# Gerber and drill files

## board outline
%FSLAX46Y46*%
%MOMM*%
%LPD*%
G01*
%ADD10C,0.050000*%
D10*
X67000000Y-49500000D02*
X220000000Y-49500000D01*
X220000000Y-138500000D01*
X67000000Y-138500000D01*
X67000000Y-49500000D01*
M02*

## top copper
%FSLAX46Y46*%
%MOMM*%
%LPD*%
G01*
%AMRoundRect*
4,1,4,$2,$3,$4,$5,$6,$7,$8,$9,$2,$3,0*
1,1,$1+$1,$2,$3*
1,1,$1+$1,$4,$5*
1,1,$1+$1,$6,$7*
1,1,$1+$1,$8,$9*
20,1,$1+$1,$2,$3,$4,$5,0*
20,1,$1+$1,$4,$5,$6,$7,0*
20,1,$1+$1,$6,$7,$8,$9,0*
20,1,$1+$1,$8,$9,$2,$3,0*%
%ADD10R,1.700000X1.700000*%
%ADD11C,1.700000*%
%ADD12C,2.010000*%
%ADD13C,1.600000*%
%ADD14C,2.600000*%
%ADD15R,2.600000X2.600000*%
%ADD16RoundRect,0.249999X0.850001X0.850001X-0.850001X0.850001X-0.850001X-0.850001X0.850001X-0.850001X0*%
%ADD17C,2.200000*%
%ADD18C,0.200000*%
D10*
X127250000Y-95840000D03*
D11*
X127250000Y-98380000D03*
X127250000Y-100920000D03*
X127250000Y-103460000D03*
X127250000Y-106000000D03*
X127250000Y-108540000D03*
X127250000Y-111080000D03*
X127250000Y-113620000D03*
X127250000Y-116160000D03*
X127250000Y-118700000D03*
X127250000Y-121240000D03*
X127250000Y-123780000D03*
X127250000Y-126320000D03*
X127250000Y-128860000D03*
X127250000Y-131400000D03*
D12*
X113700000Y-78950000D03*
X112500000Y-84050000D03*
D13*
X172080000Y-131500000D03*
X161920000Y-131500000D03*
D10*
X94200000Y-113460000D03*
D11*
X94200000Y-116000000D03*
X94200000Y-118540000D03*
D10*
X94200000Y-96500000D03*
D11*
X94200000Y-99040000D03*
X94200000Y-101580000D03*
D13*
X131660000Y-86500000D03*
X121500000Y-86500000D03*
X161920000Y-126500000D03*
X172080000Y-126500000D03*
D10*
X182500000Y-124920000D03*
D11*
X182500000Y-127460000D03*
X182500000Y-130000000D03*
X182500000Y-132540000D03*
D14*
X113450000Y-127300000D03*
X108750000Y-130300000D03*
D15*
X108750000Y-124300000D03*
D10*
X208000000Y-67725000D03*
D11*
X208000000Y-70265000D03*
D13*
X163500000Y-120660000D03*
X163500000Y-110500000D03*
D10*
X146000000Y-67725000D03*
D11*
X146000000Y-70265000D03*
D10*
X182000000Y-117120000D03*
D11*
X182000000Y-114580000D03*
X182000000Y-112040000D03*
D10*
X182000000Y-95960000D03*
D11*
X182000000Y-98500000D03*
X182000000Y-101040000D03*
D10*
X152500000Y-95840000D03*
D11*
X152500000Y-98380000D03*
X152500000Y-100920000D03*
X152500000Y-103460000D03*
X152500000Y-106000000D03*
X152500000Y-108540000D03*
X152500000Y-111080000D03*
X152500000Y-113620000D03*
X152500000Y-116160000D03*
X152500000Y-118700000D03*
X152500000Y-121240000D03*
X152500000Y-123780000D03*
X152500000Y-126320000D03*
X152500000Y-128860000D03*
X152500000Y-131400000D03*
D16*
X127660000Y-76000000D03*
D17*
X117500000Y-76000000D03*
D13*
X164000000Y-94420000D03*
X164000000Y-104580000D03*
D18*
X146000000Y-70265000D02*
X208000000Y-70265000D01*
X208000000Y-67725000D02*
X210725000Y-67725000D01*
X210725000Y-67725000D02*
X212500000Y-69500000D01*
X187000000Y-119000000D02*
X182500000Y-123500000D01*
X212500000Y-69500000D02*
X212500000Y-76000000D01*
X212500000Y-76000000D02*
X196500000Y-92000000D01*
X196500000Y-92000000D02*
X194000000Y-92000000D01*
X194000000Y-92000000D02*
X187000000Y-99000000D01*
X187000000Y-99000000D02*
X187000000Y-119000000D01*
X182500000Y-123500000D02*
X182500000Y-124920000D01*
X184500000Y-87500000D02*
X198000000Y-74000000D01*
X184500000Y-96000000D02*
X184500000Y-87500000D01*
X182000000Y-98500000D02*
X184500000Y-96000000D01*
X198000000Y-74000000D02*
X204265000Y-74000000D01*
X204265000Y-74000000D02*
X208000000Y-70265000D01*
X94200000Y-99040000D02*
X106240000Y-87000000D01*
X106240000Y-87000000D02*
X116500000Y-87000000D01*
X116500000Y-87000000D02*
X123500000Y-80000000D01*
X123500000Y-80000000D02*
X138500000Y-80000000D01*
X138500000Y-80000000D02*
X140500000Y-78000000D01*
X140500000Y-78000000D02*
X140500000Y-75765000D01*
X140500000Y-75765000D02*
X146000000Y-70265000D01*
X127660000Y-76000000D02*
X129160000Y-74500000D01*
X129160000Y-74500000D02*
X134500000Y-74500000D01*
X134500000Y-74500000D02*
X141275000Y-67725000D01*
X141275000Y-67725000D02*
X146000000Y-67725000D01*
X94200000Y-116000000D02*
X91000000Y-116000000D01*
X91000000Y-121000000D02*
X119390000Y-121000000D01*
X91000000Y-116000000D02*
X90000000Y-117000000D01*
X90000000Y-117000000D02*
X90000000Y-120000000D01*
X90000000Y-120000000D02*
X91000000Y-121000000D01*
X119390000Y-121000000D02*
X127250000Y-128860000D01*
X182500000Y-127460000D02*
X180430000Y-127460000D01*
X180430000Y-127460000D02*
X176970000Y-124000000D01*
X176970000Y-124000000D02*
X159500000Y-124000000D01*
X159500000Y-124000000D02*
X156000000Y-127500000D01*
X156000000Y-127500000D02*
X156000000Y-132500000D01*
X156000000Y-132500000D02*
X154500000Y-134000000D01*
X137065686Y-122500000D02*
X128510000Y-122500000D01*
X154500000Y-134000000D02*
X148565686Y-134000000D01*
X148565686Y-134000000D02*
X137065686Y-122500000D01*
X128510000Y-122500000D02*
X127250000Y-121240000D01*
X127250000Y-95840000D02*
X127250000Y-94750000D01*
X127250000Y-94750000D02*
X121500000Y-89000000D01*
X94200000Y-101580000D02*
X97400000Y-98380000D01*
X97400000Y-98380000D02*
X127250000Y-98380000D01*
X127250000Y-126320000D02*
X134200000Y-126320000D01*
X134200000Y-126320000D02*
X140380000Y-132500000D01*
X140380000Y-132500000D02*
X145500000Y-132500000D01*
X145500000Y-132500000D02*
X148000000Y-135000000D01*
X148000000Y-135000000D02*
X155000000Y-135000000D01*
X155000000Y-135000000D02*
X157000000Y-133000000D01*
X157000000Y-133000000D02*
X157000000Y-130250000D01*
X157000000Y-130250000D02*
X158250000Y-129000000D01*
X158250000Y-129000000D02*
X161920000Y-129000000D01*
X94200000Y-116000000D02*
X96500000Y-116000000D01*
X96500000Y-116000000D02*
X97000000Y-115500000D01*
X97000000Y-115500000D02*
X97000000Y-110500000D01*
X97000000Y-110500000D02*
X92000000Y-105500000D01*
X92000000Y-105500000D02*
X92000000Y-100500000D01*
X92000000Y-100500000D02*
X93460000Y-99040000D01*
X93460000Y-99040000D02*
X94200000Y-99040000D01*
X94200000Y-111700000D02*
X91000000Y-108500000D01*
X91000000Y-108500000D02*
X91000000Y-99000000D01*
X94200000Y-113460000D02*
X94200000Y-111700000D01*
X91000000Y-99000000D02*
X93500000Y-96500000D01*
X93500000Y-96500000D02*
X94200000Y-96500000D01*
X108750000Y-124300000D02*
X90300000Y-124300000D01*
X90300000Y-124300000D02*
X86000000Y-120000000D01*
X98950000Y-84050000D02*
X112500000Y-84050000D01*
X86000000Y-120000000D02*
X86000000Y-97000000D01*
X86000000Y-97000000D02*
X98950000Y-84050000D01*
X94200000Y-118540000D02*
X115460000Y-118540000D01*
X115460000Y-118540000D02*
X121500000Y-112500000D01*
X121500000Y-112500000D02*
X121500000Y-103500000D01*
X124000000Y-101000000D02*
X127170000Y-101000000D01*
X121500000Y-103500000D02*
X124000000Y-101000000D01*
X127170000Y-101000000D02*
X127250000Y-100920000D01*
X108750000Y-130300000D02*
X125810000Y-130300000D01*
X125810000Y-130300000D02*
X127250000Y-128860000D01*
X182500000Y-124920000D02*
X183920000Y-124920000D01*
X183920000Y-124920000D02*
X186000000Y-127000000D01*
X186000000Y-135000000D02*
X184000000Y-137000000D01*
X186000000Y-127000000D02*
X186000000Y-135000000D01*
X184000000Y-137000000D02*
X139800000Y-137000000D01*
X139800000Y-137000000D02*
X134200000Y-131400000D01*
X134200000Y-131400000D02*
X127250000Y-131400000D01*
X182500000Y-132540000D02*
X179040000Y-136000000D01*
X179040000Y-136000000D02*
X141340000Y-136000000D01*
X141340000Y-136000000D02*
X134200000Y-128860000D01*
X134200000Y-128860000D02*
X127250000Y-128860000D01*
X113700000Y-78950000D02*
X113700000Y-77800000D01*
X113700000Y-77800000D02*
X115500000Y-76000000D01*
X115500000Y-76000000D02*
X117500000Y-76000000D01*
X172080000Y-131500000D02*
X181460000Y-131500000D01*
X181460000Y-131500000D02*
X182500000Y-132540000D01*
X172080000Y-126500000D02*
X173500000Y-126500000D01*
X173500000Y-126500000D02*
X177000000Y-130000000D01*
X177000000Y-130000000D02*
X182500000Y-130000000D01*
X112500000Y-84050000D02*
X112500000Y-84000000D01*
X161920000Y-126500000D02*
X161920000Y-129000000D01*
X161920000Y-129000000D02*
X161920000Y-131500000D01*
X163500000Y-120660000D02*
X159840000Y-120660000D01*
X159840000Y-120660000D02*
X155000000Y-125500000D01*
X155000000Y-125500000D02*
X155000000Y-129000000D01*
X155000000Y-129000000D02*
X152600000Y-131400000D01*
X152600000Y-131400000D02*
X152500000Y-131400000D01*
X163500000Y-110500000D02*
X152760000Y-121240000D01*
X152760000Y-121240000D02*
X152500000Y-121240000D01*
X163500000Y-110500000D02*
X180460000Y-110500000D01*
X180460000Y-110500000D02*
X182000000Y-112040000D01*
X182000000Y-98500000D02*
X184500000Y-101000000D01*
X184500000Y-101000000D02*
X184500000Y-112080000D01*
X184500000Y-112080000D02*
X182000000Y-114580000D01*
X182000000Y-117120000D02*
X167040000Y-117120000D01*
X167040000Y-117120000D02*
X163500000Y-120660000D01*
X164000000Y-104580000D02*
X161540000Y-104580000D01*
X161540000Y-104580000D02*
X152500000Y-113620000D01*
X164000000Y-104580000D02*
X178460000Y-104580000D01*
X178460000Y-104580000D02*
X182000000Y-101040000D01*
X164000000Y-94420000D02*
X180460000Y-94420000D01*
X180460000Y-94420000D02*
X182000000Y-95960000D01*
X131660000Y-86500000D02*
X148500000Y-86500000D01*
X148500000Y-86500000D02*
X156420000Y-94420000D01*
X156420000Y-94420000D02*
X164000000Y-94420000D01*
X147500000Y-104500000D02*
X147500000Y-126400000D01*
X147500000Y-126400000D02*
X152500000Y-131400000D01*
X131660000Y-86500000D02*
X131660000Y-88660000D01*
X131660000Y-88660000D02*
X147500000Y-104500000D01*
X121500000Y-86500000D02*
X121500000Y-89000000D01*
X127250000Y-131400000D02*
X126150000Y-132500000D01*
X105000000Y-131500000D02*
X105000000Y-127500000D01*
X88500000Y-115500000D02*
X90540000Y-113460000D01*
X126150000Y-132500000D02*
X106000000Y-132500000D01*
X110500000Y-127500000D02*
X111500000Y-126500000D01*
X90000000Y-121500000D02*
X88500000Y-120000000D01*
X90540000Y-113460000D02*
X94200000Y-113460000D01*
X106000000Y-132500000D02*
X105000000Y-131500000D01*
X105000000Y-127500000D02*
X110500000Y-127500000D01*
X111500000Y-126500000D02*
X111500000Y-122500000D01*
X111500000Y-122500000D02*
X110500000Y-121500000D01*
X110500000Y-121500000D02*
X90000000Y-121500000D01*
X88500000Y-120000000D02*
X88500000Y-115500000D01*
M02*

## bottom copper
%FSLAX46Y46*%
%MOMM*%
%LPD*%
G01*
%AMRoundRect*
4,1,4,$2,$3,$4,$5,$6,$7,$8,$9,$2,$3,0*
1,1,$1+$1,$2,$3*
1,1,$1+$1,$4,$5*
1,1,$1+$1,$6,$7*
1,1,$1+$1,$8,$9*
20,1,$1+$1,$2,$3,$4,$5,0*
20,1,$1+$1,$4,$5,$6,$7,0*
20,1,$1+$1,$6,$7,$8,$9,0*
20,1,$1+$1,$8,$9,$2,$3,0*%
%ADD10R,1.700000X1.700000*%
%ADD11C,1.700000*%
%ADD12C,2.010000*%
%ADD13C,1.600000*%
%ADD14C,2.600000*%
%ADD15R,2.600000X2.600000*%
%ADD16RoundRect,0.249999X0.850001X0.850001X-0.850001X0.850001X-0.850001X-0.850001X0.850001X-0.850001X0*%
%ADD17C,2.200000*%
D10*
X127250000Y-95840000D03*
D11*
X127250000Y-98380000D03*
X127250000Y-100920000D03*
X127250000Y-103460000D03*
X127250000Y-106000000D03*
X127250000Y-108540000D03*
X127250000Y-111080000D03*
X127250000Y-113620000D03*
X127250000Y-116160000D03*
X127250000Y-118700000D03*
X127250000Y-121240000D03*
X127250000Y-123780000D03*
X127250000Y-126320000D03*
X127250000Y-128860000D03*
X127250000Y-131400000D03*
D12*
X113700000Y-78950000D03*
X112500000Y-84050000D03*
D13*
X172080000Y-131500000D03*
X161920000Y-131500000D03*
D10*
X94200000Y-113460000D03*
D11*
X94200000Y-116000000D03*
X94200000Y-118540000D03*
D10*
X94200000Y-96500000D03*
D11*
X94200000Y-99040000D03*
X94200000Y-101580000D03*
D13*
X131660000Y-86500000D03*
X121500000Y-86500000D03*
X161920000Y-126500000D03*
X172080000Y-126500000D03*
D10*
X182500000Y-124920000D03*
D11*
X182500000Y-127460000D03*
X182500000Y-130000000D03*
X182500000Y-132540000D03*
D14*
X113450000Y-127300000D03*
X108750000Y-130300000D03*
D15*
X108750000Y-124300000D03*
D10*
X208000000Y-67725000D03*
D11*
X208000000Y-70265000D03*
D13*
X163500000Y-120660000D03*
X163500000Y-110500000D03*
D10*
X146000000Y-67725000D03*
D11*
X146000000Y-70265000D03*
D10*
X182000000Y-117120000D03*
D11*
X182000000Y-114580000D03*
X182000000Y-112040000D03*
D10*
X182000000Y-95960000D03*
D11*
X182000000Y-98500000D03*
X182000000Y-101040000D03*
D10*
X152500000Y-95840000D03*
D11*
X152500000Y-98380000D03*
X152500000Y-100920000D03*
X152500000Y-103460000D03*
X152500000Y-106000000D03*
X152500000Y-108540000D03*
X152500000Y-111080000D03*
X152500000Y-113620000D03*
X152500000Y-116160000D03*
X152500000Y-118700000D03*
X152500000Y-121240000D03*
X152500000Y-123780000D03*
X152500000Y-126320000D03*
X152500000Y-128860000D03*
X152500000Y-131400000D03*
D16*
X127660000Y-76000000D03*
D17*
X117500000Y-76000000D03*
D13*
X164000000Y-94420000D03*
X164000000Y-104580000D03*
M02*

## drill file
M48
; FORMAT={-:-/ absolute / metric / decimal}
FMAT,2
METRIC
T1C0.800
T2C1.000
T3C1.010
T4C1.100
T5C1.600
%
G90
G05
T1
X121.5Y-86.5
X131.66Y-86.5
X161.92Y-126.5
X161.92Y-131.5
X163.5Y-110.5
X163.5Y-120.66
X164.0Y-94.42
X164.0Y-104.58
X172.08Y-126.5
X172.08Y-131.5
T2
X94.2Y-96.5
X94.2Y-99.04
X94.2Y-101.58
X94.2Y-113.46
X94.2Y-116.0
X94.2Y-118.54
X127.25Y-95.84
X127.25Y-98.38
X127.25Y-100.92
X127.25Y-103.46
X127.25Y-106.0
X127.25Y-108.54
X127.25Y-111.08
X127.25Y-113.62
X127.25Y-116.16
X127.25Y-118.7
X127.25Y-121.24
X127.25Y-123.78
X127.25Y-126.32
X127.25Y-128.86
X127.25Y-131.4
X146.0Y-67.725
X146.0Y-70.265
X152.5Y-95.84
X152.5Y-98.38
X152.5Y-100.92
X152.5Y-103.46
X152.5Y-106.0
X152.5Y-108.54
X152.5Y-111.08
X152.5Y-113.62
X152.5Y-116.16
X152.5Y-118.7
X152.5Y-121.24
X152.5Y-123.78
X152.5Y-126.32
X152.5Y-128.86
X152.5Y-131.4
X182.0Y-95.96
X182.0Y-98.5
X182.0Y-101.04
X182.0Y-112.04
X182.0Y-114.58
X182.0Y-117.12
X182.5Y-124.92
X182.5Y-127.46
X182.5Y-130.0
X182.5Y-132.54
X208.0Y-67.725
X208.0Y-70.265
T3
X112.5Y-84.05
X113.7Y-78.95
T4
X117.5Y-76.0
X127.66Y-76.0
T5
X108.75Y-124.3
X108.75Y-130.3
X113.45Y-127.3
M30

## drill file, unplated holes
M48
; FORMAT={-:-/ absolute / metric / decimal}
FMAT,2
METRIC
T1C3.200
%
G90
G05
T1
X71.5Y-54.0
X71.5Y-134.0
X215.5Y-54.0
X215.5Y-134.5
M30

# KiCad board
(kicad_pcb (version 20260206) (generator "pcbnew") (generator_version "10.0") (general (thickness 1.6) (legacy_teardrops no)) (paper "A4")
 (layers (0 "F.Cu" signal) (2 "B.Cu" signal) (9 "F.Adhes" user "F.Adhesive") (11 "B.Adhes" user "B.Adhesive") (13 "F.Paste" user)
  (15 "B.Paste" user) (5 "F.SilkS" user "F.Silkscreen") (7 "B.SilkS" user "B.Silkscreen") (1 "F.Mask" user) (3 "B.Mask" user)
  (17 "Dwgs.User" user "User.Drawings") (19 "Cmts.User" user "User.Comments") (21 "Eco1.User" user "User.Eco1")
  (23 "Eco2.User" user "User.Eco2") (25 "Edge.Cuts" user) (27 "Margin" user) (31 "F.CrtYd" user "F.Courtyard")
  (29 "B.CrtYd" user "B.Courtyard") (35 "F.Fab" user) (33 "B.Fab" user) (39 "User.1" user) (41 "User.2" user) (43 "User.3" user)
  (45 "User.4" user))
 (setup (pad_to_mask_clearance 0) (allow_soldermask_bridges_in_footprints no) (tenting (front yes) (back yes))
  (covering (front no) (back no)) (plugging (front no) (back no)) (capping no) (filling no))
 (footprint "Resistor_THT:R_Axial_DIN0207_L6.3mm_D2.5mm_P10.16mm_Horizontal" (layer "F.Cu") (at 161.92 126.5)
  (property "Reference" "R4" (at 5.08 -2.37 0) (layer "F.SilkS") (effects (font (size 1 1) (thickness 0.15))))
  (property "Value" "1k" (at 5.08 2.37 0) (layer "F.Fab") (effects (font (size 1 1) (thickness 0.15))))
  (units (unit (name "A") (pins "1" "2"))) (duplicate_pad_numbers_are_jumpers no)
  (pad "1" thru_hole circle (at 0 0) (size 1.6 1.6) (drill 0.8) (layers "*.Cu" "*.Mask") (remove_unused_layers no) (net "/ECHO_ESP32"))
  (pad "2" thru_hole circle (at 10.16 0) (size 1.6 1.6) (drill 0.8) (layers "*.Cu" "*.Mask") (remove_unused_layers no) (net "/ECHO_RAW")))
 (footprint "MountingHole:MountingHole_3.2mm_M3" (layer "F.Cu") (at 215.5 134.5)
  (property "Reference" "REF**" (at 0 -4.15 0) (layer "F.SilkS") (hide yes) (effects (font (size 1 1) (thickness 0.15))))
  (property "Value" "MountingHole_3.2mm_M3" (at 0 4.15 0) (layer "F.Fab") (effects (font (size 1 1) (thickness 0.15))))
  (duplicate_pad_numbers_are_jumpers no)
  (pad "" np_thru_hole circle (at 0 0) (size 3.2 3.2) (drill 3.2) (layers "*.Cu" "*.Mask")))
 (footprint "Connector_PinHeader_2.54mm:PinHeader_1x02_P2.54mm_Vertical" (layer "F.Cu") (at 208 67.725)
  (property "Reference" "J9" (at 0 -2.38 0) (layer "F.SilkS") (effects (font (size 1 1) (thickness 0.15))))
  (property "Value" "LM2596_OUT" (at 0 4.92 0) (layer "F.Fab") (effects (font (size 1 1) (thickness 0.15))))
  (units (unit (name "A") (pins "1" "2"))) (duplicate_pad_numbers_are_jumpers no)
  (pad "1" thru_hole rect (at 0 0) (size 1.7 1.7) (drill 1) (layers "*.Cu" "*.Mask") (remove_unused_layers no) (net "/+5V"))
  (pad "2" thru_hole circle (at 0 2.54) (size 1.7 1.7) (drill 1) (layers "*.Cu" "*.Mask") (remove_unused_layers no) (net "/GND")))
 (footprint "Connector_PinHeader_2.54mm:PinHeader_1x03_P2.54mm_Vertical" (layer "F.Cu") (at 94.2 113.46)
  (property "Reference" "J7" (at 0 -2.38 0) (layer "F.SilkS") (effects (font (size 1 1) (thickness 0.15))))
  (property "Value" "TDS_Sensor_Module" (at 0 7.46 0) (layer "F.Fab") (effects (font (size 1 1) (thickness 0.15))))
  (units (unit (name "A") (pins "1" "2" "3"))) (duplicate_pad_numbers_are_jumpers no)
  (pad "1" thru_hole rect (at 0 0) (size 1.7 1.7) (drill 1) (layers "*.Cu" "*.Mask") (remove_unused_layers no) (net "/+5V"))
  (pad "2" thru_hole circle (at 0 2.54) (size 1.7 1.7) (drill 1) (layers "*.Cu" "*.Mask") (remove_unused_layers no) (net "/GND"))
  (pad "3" thru_hole circle (at 0 5.08) (size 1.7 1.7) (drill 1) (layers "*.Cu" "*.Mask") (remove_unused_layers no) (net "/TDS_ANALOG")))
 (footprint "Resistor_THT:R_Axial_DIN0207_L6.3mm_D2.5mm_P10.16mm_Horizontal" (layer "F.Cu") (at 131.66 86.5 180)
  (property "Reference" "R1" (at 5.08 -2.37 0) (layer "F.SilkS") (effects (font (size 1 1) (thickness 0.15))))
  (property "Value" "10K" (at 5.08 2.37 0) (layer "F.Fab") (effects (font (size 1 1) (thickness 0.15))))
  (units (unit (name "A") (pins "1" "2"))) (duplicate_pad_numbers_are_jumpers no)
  (pad "1" thru_hole circle (at 0 0 180) (size 1.6 1.6) (drill 0.8) (layers "*.Cu" "*.Mask") (remove_unused_layers no) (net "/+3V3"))
  (pad "2" thru_hole circle (at 10.16 0 180) (size 1.6 1.6) (drill 0.8) (layers "*.Cu" "*.Mask") (remove_unused_layers no) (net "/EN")))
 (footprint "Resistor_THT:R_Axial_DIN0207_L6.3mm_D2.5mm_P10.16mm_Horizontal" (layer "F.Cu") (at 163.5 120.66 90)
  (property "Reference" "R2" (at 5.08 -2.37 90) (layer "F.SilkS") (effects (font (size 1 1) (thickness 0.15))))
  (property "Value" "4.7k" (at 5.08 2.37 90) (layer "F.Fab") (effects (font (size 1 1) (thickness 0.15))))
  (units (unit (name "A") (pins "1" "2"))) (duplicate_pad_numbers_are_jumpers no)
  (pad "1" thru_hole circle (at 0 0 90) (size 1.6 1.6) (drill 0.8) (layers "*.Cu" "*.Mask") (remove_unused_layers no) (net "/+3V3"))
  (pad "2" thru_hole circle (at 10.16 0 90) (size 1.6 1.6) (drill 0.8) (layers "*.Cu" "*.Mask") (remove_unused_layers no)
   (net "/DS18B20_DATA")))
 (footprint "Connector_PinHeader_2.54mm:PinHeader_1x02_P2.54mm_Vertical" (layer "F.Cu") (at 146 67.725)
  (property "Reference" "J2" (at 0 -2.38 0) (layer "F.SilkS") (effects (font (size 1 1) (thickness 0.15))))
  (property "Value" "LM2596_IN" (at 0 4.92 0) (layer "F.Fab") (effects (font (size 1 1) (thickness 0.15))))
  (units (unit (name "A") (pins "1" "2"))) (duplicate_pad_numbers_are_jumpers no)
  (pad "1" thru_hole rect (at 0 0) (size 1.7 1.7) (drill 1) (layers "*.Cu" "*.Mask") (remove_unused_layers no) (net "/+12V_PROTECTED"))
  (pad "2" thru_hole circle (at 0 2.54) (size 1.7 1.7) (drill 1) (layers "*.Cu" "*.Mask") (remove_unused_layers no) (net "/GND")))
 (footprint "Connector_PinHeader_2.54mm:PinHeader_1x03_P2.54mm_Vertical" (layer "F.Cu") (at 182 117.12 180)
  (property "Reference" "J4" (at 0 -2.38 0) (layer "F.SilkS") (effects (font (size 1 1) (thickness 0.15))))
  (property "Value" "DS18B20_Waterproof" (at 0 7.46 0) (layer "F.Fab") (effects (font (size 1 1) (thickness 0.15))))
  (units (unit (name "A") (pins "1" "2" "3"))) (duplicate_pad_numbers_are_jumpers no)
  (pad "1" thru_hole rect (at 0 0 180) (size 1.7 1.7) (drill 1) (layers "*.Cu" "*.Mask") (remove_unused_layers no) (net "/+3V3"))
  (pad "2" thru_hole circle (at 0 2.54 180) (size 1.7 1.7) (drill 1) (layers "*.Cu" "*.Mask") (remove_unused_layers no) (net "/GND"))
  (pad "3" thru_hole circle (at 0 5.08 180) (size 1.7 1.7) (drill 1) (layers "*.Cu" "*.Mask") (remove_unused_layers no)
   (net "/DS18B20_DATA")))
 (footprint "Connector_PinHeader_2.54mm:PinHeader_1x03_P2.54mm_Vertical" (layer "F.Cu") (at 94.2 96.5)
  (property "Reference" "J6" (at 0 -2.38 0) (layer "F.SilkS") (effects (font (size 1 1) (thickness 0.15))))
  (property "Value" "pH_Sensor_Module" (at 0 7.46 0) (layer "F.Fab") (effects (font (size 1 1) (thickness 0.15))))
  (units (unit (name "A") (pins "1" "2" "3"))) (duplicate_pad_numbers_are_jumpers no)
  (pad "1" thru_hole rect (at 0 0) (size 1.7 1.7) (drill 1) (layers "*.Cu" "*.Mask") (remove_unused_layers no) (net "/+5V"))
  (pad "2" thru_hole circle (at 0 2.54) (size 1.7 1.7) (drill 1) (layers "*.Cu" "*.Mask") (remove_unused_layers no) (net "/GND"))
  (pad "3" thru_hole circle (at 0 5.08) (size 1.7 1.7) (drill 1) (layers "*.Cu" "*.Mask") (remove_unused_layers no) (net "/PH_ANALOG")))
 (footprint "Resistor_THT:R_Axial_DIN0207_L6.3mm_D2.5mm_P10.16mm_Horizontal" (layer "F.Cu") (at 161.92 131.5)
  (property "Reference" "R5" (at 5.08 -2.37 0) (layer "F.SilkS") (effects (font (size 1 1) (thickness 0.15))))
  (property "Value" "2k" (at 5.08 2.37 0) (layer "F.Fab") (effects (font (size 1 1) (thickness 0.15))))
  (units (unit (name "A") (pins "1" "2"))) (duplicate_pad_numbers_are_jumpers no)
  (pad "1" thru_hole circle (at 0 0) (size 1.6 1.6) (drill 0.8) (layers "*.Cu" "*.Mask") (remove_unused_layers no) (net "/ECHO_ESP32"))
  (pad "2" thru_hole circle (at 10.16 0) (size 1.6 1.6) (drill 0.8) (layers "*.Cu" "*.Mask") (remove_unused_layers no) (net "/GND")))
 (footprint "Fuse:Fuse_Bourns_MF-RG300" (layer "F.Cu") (at 113.7 78.95 -90)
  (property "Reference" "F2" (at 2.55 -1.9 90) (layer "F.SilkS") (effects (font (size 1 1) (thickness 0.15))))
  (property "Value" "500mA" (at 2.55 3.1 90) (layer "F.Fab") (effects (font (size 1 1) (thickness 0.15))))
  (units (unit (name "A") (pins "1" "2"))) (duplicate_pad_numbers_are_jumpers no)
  (pad "1" thru_hole circle (at 0 0 270) (size 2.01 2.01) (drill 1.01) (layers "*.Cu" "*.Mask") (remove_unused_layers no)
   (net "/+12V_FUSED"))
  (pad "2" thru_hole circle (at 5.1 1.2 270) (size 2.01 2.01) (drill 1.01) (layers "*.Cu" "*.Mask") (remove_unused_layers no)
   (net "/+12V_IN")))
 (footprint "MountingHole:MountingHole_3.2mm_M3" (layer "F.Cu") (at 71.5 134)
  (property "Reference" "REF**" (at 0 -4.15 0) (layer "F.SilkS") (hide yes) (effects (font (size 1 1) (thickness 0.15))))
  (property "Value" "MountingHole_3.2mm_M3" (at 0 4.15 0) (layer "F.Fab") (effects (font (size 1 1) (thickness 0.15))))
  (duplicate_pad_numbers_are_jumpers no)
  (pad "" np_thru_hole circle (at 0 0) (size 3.2 3.2) (drill 3.2) (layers "*.Cu" "*.Mask")))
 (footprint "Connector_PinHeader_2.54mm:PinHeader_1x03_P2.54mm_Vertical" (layer "F.Cu") (at 182 95.96)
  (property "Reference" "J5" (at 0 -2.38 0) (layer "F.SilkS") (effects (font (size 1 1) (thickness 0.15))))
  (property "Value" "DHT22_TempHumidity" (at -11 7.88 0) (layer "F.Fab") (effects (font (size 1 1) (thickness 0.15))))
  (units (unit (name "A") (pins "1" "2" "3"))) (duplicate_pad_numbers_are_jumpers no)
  (pad "1" thru_hole rect (at 0 0) (size 1.7 1.7) (drill 1) (layers "*.Cu" "*.Mask") (remove_unused_layers no) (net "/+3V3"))
  (pad "2" thru_hole circle (at 0 2.54) (size 1.7 1.7) (drill 1) (layers "*.Cu" "*.Mask") (remove_unused_layers no) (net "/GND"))
  (pad "3" thru_hole circle (at 0 5.08) (size 1.7 1.7) (drill 1) (layers "*.Cu" "*.Mask") (remove_unused_layers no) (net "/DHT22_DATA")))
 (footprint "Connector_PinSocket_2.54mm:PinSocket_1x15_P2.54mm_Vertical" (layer "F.Cu") (at 127.25 95.84)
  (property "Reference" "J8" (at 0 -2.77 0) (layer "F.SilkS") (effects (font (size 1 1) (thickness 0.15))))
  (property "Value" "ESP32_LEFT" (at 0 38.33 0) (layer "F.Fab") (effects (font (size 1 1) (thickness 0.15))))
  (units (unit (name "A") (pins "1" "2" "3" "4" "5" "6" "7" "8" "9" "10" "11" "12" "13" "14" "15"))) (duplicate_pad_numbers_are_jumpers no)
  (pad "1" thru_hole rect (at 0 0) (size 1.7 1.7) (drill 1) (layers "*.Cu" "*.Mask") (remove_unused_layers no) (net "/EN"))
  (pad "2" thru_hole circle (at 0 2.54) (size 1.7 1.7) (drill 1) (layers "*.Cu" "*.Mask") (remove_unused_layers no) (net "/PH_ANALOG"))
  (pad "3" thru_hole circle (at 0 5.08) (size 1.7 1.7) (drill 1) (layers "*.Cu" "*.Mask") (remove_unused_layers no) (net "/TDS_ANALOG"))
  (pad "4" thru_hole circle (at 0 7.62) (size 1.7 1.7) (drill 1) (layers "*.Cu" "*.Mask") (remove_unused_layers no)
   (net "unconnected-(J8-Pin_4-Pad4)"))
  (pad "5" thru_hole circle (at 0 10.16) (size 1.7 1.7) (drill 1) (layers "*.Cu" "*.Mask") (remove_unused_layers no)
   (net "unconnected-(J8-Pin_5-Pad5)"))
  (pad "6" thru_hole circle (at 0 12.7) (size 1.7 1.7) (drill 1) (layers "*.Cu" "*.Mask") (remove_unused_layers no)
   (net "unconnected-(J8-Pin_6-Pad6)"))
  (pad "7" thru_hole circle (at 0 15.24) (size 1.7 1.7) (drill 1) (layers "*.Cu" "*.Mask") (remove_unused_layers no)
   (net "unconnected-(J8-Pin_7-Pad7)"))
  (pad "8" thru_hole circle (at 0 17.78) (size 1.7 1.7) (drill 1) (layers "*.Cu" "*.Mask") (remove_unused_layers no)
   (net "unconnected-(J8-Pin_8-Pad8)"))
  (pad "9" thru_hole circle (at 0 20.32) (size 1.7 1.7) (drill 1) (layers "*.Cu" "*.Mask") (remove_unused_layers no)
   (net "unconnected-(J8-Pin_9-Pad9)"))
  (pad "10" thru_hole circle (at 0 22.86) (size 1.7 1.7) (drill 1) (layers "*.Cu" "*.Mask") (remove_unused_layers no)
   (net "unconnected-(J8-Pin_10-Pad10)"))
  (pad "11" thru_hole circle (at 0 25.4) (size 1.7 1.7) (drill 1) (layers "*.Cu" "*.Mask") (remove_unused_layers no) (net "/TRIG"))
  (pad "12" thru_hole circle (at 0 27.94) (size 1.7 1.7) (drill 1) (layers "*.Cu" "*.Mask") (remove_unused_layers no)
   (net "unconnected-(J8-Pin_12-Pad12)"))
  (pad "13" thru_hole circle (at 0 30.48) (size 1.7 1.7) (drill 1) (layers "*.Cu" "*.Mask") (remove_unused_layers no) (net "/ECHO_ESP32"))
  (pad "14" thru_hole circle (at 0 33.02) (size 1.7 1.7) (drill 1) (layers "*.Cu" "*.Mask") (remove_unused_layers no) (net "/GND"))
  (pad "15" thru_hole circle (at 0 35.56) (size 1.7 1.7) (drill 1) (layers "*.Cu" "*.Mask") (remove_unused_layers no) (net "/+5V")))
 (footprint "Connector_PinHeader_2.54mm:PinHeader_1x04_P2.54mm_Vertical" (layer "F.Cu") (at 182.5 124.92)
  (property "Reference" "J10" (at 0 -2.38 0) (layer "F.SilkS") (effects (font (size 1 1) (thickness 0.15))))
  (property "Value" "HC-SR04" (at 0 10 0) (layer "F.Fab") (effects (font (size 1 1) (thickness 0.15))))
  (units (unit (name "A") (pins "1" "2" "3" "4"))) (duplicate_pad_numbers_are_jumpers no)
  (pad "1" thru_hole rect (at 0 0) (size 1.7 1.7) (drill 1) (layers "*.Cu" "*.Mask") (remove_unused_layers no) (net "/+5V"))
  (pad "2" thru_hole circle (at 0 2.54) (size 1.7 1.7) (drill 1) (layers "*.Cu" "*.Mask") (remove_unused_layers no) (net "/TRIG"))
  (pad "3" thru_hole circle (at 0 5.08) (size 1.7 1.7) (drill 1) (layers "*.Cu" "*.Mask") (remove_unused_layers no) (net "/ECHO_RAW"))
  (pad "4" thru_hole circle (at 0 7.62) (size 1.7 1.7) (drill 1) (layers "*.Cu" "*.Mask") (remove_unused_layers no) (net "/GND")))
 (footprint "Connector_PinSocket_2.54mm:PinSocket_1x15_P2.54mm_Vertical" (layer "F.Cu") (at 152.5 95.84)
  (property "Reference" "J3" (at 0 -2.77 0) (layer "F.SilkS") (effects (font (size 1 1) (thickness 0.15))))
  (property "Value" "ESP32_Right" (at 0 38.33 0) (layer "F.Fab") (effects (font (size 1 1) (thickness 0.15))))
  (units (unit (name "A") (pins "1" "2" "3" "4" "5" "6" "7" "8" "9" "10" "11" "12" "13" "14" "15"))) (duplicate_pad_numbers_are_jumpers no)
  (pad "1" thru_hole rect (at 0 0) (size 1.7 1.7) (drill 1) (layers "*.Cu" "*.Mask") (remove_unused_layers no)
   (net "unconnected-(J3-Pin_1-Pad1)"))
  (pad "2" thru_hole circle (at 0 2.54) (size 1.7 1.7) (drill 1) (layers "*.Cu" "*.Mask") (remove_unused_layers no)
   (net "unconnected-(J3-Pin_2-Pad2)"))
  (pad "3" thru_hole circle (at 0 5.08) (size 1.7 1.7) (drill 1) (layers "*.Cu" "*.Mask") (remove_unused_layers no)
   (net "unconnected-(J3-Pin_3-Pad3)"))
  (pad "4" thru_hole circle (at 0 7.62) (size 1.7 1.7) (drill 1) (layers "*.Cu" "*.Mask") (remove_unused_layers no)
   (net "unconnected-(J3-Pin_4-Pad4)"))
  (pad "5" thru_hole circle (at 0 10.16) (size 1.7 1.7) (drill 1) (layers "*.Cu" "*.Mask") (remove_unused_layers no)
   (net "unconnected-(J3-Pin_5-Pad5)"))
  (pad "6" thru_hole circle (at 0 12.7) (size 1.7 1.7) (drill 1) (layers "*.Cu" "*.Mask") (remove_unused_layers no)
   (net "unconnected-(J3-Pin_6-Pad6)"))
  (pad "7" thru_hole circle (at 0 15.24) (size 1.7 1.7) (drill 1) (layers "*.Cu" "*.Mask") (remove_unused_layers no)
   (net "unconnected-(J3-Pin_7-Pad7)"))
  (pad "8" thru_hole circle (at 0 17.78) (size 1.7 1.7) (drill 1) (layers "*.Cu" "*.Mask") (remove_unused_layers no) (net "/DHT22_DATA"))
  (pad "9" thru_hole circle (at 0 20.32) (size 1.7 1.7) (drill 1) (layers "*.Cu" "*.Mask") (remove_unused_layers no)
   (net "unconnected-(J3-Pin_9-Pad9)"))
  (pad "10" thru_hole circle (at 0 22.86) (size 1.7 1.7) (drill 1) (layers "*.Cu" "*.Mask") (remove_unused_layers no)
   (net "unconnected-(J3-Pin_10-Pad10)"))
  (pad "11" thru_hole circle (at 0 25.4) (size 1.7 1.7) (drill 1) (layers "*.Cu" "*.Mask") (remove_unused_layers no) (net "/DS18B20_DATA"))
  (pad "12" thru_hole circle (at 0 27.94) (size 1.7 1.7) (drill 1) (layers "*.Cu" "*.Mask") (remove_unused_layers no)
   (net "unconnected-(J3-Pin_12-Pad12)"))
  (pad "13" thru_hole circle (at 0 30.48) (size 1.7 1.7) (drill 1) (layers "*.Cu" "*.Mask") (remove_unused_layers no)
   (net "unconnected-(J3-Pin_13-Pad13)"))
  (pad "14" thru_hole circle (at 0 33.02) (size 1.7 1.7) (drill 1) (layers "*.Cu" "*.Mask") (remove_unused_layers no)
   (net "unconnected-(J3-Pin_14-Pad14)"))
  (pad "15" thru_hole circle (at 0 35.56) (size 1.7 1.7) (drill 1) (layers "*.Cu" "*.Mask") (remove_unused_layers no) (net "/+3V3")))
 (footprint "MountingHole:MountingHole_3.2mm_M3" (layer "F.Cu") (at 215.5 54)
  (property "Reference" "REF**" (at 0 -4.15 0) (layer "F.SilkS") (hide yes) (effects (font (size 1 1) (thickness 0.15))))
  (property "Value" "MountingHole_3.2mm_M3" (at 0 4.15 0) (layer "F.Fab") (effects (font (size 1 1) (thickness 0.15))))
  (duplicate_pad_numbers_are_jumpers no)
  (pad "" np_thru_hole circle (at 0 0) (size 3.2 3.2) (drill 3.2) (layers "*.Cu" "*.Mask")))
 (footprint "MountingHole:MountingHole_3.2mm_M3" (layer "F.Cu") (at 71.5 54)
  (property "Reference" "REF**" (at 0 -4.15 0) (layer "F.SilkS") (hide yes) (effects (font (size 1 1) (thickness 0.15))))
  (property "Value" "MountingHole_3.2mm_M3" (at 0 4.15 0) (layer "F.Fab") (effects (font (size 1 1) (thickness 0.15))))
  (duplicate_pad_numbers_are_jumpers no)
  (pad "" np_thru_hole circle (at 0 0) (size 3.2 3.2) (drill 3.2) (layers "*.Cu" "*.Mask")))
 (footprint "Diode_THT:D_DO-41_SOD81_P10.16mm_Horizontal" (layer "F.Cu") (at 127.66 76 180)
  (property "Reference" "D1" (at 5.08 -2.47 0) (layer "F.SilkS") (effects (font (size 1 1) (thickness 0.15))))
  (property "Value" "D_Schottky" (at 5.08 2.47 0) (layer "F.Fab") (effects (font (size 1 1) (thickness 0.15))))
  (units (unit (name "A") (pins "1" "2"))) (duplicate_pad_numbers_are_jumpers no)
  (pad "1" thru_hole roundrect (at 0 0 180) (size 2.2 2.2) (drill 1.1) (layers "*.Cu" "*.Mask") (remove_unused_layers no)
   (roundrect_rratio 0.113636) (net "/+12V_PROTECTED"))
  (pad "2" thru_hole circle (at 10.16 0 180) (size 2.2 2.2) (drill 1.1) (layers "*.Cu" "*.Mask") (remove_unused_layers no)
   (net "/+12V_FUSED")))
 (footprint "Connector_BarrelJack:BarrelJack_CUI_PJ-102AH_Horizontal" (layer "F.Cu") (at 108.75 124.3)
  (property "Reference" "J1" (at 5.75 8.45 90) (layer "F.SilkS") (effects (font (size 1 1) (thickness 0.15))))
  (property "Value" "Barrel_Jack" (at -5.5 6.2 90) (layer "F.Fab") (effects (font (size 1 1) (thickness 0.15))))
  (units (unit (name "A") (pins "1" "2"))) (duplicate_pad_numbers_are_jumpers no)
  (pad "1" thru_hole rect (at 0 0) (size 2.6 2.6) (drill 1.6) (layers "*.Cu" "*.Mask") (remove_unused_layers no) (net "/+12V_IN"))
  (pad "2" thru_hole circle (at 0 6) (size 2.6 2.6) (drill 1.6) (layers "*.Cu" "*.Mask") (remove_unused_layers no) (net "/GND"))
  (pad "3" thru_hole circle (at 4.7 3) (size 2.6 2.6) (drill 1.6) (layers "*.Cu" "*.Mask") (remove_unused_layers no)))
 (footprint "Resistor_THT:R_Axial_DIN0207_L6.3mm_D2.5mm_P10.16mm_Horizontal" (layer "F.Cu") (at 164 94.42 -90)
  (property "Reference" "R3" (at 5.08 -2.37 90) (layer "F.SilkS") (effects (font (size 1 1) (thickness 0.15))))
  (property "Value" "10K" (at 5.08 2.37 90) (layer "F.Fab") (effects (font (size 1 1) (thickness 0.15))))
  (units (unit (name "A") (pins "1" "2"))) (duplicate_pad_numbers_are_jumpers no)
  (pad "1" thru_hole circle (at 0 0 270) (size 1.6 1.6) (drill 0.8) (layers "*.Cu" "*.Mask") (remove_unused_layers no) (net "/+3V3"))
  (pad "2" thru_hole circle (at 10.16 0 270) (size 1.6 1.6) (drill 0.8) (layers "*.Cu" "*.Mask") (remove_unused_layers no)
   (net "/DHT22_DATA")))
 (gr_rect (start 67 49.5) (end 220 138.5) (stroke (width 0.05) (type default)) (fill no) (layer "Edge.Cuts"))
 (segment (start 110.5 127.5) (end 111.5 126.5) (width 0.2) (layer "F.Cu") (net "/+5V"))
 (segment (start 212.5 69.5) (end 212.5 76) (width 0.2) (layer "F.Cu") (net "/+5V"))
 (segment (start 93.5 96.5) (end 94.2 96.5) (width 0.2) (layer "F.Cu") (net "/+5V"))
 (segment (start 111.5 122.5) (end 110.5 121.5) (width 0.2) (layer "F.Cu") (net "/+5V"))
 (segment (start 111.5 126.5) (end 111.5 122.5) (width 0.2) (layer "F.Cu") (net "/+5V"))
 (segment (start 186 135) (end 184 137) (width 0.2) (layer "F.Cu") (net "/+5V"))
 (segment (start 186 127) (end 186 135) (width 0.2) (layer "F.Cu") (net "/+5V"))
 (segment (start 139.8 137) (end 134.2 131.4) (width 0.2) (layer "F.Cu") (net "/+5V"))
 (segment (start 126.15 132.5) (end 106 132.5) (width 0.2) (layer "F.Cu") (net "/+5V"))
 (segment (start 212.5 76) (end 196.5 92) (width 0.2) (layer "F.Cu") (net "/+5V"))
 (segment (start 94.2 113.46) (end 94.2 111.7) (width 0.2) (layer "F.Cu") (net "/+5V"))
 (segment (start 105 131.5) (end 105 127.5) (width 0.2) (layer "F.Cu") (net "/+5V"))
 (segment (start 184 137) (end 139.8 137) (width 0.2) (layer "F.Cu") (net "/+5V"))
 (segment (start 88.5 115.5) (end 90.54 113.46) (width 0.2) (layer "F.Cu") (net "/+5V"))
 (segment (start 187 99) (end 187 119) (width 0.2) (layer "F.Cu") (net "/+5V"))
 (segment (start 90.54 113.46) (end 94.2 113.46) (width 0.2) (layer "F.Cu") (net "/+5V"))
 (segment (start 90 121.5) (end 88.5 120) (width 0.2) (layer "F.Cu") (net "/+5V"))
 (segment (start 94.2 111.7) (end 91 108.5) (width 0.2) (layer "F.Cu") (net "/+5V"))
 (segment (start 187 119) (end 182.5 123.5) (width 0.2) (layer "F.Cu") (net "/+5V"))
 (segment (start 91 99) (end 93.5 96.5) (width 0.2) (layer "F.Cu") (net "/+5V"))
 (segment (start 182.5 124.92) (end 183.92 124.92) (width 0.2) (layer "F.Cu") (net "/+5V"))
 (segment (start 91 108.5) (end 91 99) (width 0.2) (layer "F.Cu") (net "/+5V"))
 (segment (start 208 67.725) (end 210.725 67.725) (width 0.2) (layer "F.Cu") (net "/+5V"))
 (segment (start 110.5 121.5) (end 90 121.5) (width 0.2) (layer "F.Cu") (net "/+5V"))
 (segment (start 127.25 131.4) (end 126.15 132.5) (width 0.2) (layer "F.Cu") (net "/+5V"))
 (segment (start 105 127.5) (end 110.5 127.5) (width 0.2) (layer "F.Cu") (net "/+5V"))
 (segment (start 134.2 131.4) (end 127.25 131.4) (width 0.2) (layer "F.Cu") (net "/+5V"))
 (segment (start 196.5 92) (end 194 92) (width 0.2) (layer "F.Cu") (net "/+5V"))
 (segment (start 106 132.5) (end 105 131.5) (width 0.2) (layer "F.Cu") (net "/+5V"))
 (segment (start 194 92) (end 187 99) (width 0.2) (layer "F.Cu") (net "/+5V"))
 (segment (start 210.725 67.725) (end 212.5 69.5) (width 0.2) (layer "F.Cu") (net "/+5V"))
 (segment (start 88.5 120) (end 88.5 115.5) (width 0.2) (layer "F.Cu") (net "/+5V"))
 (segment (start 183.92 124.92) (end 186 127) (width 0.2) (layer "F.Cu") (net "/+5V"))
 (segment (start 182.5 123.5) (end 182.5 124.92) (width 0.2) (layer "F.Cu") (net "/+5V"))
 (segment (start 91 116) (end 90 117) (width 0.2) (layer "F.Cu") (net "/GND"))
 (segment (start 141.34 136) (end 134.2 128.86) (width 0.2) (layer "F.Cu") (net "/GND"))
 (segment (start 90 117) (end 90 120) (width 0.2) (layer "F.Cu") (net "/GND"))
 (segment (start 97 115.5) (end 97 110.5) (width 0.2) (layer "F.Cu") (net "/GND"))
 (segment (start 94.2 116) (end 91 116) (width 0.2) (layer "F.Cu") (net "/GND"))
 (segment (start 134.2 128.86) (end 127.25 128.86) (width 0.2) (layer "F.Cu") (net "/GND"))
 (segment (start 184.5 87.5) (end 198 74) (width 0.2) (layer "F.Cu") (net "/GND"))
 (segment (start 94.2 99.04) (end 106.24 87) (width 0.2) (layer "F.Cu") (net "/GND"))
 (segment (start 108.75 130.3) (end 125.81 130.3) (width 0.2) (layer "F.Cu") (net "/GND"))
 (segment (start 204.265 74) (end 208 70.265) (width 0.2) (layer "F.Cu") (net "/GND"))
 (segment (start 181.46 131.5) (end 182.5 132.54) (width 0.2) (layer "F.Cu") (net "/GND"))
 (segment (start 90 120) (end 91 121) (width 0.2) (layer "F.Cu") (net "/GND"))
 (segment (start 93.46 99.04) (end 94.2 99.04) (width 0.2) (layer "F.Cu") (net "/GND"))
 (segment (start 179.04 136) (end 141.34 136) (width 0.2) (layer "F.Cu") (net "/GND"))
 (segment (start 182.5 132.54) (end 179.04 136) (width 0.2) (layer "F.Cu") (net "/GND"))
 (segment (start 123.5 80) (end 138.5 80) (width 0.2) (layer "F.Cu") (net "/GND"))
 (segment (start 92 100.5) (end 93.46 99.04) (width 0.2) (layer "F.Cu") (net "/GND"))
 (segment (start 184.5 96) (end 184.5 87.5) (width 0.2) (layer "F.Cu") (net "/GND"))
 (segment (start 140.5 78) (end 140.5 75.765) (width 0.2) (layer "F.Cu") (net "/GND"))
 (segment (start 94.2 116) (end 96.5 116) (width 0.2) (layer "F.Cu") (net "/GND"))
 (segment (start 96.5 116) (end 97 115.5) (width 0.2) (layer "F.Cu") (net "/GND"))
 (segment (start 198 74) (end 204.265 74) (width 0.2) (layer "F.Cu") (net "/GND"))
 (segment (start 119.39 121) (end 127.25 128.86) (width 0.2) (layer "F.Cu") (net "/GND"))
 (segment (start 138.5 80) (end 140.5 78) (width 0.2) (layer "F.Cu") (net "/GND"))
 (segment (start 125.81 130.3) (end 127.25 128.86) (width 0.2) (layer "F.Cu") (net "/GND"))
 (segment (start 140.5 75.765) (end 146 70.265) (width 0.2) (layer "F.Cu") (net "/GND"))
 (segment (start 92 105.5) (end 92 100.5) (width 0.2) (layer "F.Cu") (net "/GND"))
 (segment (start 116.5 87) (end 123.5 80) (width 0.2) (layer "F.Cu") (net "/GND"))
 (segment (start 146 70.265) (end 208 70.265) (width 0.2) (layer "F.Cu") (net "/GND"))
 (segment (start 184.5 101) (end 184.5 112.08) (width 0.2) (layer "F.Cu") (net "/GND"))
 (segment (start 182 98.5) (end 184.5 101) (width 0.2) (layer "F.Cu") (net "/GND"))
 (segment (start 91 121) (end 119.39 121) (width 0.2) (layer "F.Cu") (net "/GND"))
 (segment (start 182 98.5) (end 184.5 96) (width 0.2) (layer "F.Cu") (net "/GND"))
 (segment (start 97 110.5) (end 92 105.5) (width 0.2) (layer "F.Cu") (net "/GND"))
 (segment (start 172.08 131.5) (end 181.46 131.5) (width 0.2) (layer "F.Cu") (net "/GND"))
 (segment (start 184.5 112.08) (end 182 114.58) (width 0.2) (layer "F.Cu") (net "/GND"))
 (segment (start 106.24 87) (end 116.5 87) (width 0.2) (layer "F.Cu") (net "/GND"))
 (segment (start 115.46 118.54) (end 121.5 112.5) (width 0.2) (layer "F.Cu") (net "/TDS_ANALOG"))
 (segment (start 94.2 118.54) (end 115.46 118.54) (width 0.2) (layer "F.Cu") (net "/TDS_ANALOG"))
 (segment (start 124 101) (end 127.17 101) (width 0.2) (layer "F.Cu") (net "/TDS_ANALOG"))
 (segment (start 127.17 101) (end 127.25 100.92) (width 0.2) (layer "F.Cu") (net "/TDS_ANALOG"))
 (segment (start 121.5 103.5) (end 124 101) (width 0.2) (layer "F.Cu") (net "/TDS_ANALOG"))
 (segment (start 121.5 112.5) (end 121.5 103.5) (width 0.2) (layer "F.Cu") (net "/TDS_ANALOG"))
 (segment (start 155 125.5) (end 155 129) (width 0.2) (layer "F.Cu") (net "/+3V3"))
 (segment (start 152.6 131.4) (end 152.5 131.4) (width 0.2) (layer "F.Cu") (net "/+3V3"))
 (segment (start 147.5 104.5) (end 147.5 126.4) (width 0.2) (layer "F.Cu") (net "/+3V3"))
 (segment (start 180.46 94.42) (end 182 95.96) (width 0.2) (layer "F.Cu") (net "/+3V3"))
 (segment (start 156.42 94.42) (end 164 94.42) (width 0.2) (layer "F.Cu") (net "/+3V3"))
 (segment (start 148.5 86.5) (end 156.42 94.42) (width 0.2) (layer "F.Cu") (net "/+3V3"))
 (segment (start 147.5 126.4) (end 152.5 131.4) (width 0.2) (layer "F.Cu") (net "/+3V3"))
 (segment (start 163.5 120.66) (end 159.84 120.66) (width 0.2) (layer "F.Cu") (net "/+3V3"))
 (segment (start 131.66 86.5) (end 148.5 86.5) (width 0.2) (layer "F.Cu") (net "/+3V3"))
 (segment (start 159.84 120.66) (end 155 125.5) (width 0.2) (layer "F.Cu") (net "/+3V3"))
 (segment (start 131.66 86.5) (end 131.66 88.66) (width 0.2) (layer "F.Cu") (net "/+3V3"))
 (segment (start 131.66 88.66) (end 147.5 104.5) (width 0.2) (layer "F.Cu") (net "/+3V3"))
 (segment (start 164 94.42) (end 180.46 94.42) (width 0.2) (layer "F.Cu") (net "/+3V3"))
 (segment (start 155 129) (end 152.6 131.4) (width 0.2) (layer "F.Cu") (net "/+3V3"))
 (segment (start 167.04 117.12) (end 163.5 120.66) (width 0.2) (layer "F.Cu") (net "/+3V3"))
 (segment (start 182 117.12) (end 167.04 117.12) (width 0.2) (layer "F.Cu") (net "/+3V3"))
 (segment (start 121.5 86.5) (end 121.5 89) (width 0.2) (layer "F.Cu") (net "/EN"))
 (segment (start 127.25 95.84) (end 127.25 94.75) (width 0.2) (layer "F.Cu") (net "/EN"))
 (segment (start 127.25 94.75) (end 121.5 89) (width 0.2) (layer "F.Cu") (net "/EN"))
 (segment (start 152.76 121.24) (end 152.5 121.24) (width 0.2) (layer "F.Cu") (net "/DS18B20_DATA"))
 (segment (start 180.46 110.5) (end 182 112.04) (width 0.2) (layer "F.Cu") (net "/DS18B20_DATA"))
 (segment (start 163.5 110.5) (end 180.46 110.5) (width 0.2) (layer "F.Cu") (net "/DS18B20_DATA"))
 (segment (start 163.5 110.5) (end 152.76 121.24) (width 0.2) (layer "F.Cu") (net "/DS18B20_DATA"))
 (segment (start 141.275 67.725) (end 146 67.725) (width 0.2) (layer "F.Cu") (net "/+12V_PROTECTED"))
 (segment (start 134.5 74.5) (end 141.275 67.725) (width 0.2) (layer "F.Cu") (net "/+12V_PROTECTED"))
 (segment (start 127.66 76) (end 129.16 74.5) (width 0.2) (layer "F.Cu") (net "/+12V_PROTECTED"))
 (segment (start 129.16 74.5) (end 134.5 74.5) (width 0.2) (layer "F.Cu") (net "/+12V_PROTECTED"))
 (segment (start 97.4 98.38) (end 127.25 98.38) (width 0.2) (layer "F.Cu") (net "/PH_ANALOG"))
 (segment (start 94.2 101.58) (end 97.4 98.38) (width 0.2) (layer "F.Cu") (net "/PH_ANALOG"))
 (segment (start 115.5 76) (end 117.5 76) (width 0.2) (layer "F.Cu") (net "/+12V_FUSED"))
 (segment (start 113.7 78.95) (end 113.7 77.8) (width 0.2) (layer "F.Cu") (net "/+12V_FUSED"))
 (segment (start 113.7 77.8) (end 115.5 76) (width 0.2) (layer "F.Cu") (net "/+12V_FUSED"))
 (segment (start 112.5 84.05) (end 112.5 84) (width 0.2) (layer "F.Cu") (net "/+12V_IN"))
 (segment (start 98.95 84.05) (end 112.5 84.05) (width 0.2) (layer "F.Cu") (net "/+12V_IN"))
 (segment (start 108.75 124.3) (end 90.3 124.3) (width 0.2) (layer "F.Cu") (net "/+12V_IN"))
 (segment (start 90.3 124.3) (end 86 120) (width 0.2) (layer "F.Cu") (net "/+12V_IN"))
 (segment (start 86 97) (end 98.95 84.05) (width 0.2) (layer "F.Cu") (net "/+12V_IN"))
 (segment (start 86 120) (end 86 97) (width 0.2) (layer "F.Cu") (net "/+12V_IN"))
 (segment (start 178.46 104.58) (end 182 101.04) (width 0.2) (layer "F.Cu") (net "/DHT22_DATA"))
 (segment (start 161.54 104.58) (end 152.5 113.62) (width 0.2) (layer "F.Cu") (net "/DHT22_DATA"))
 (segment (start 164 104.58) (end 178.46 104.58) (width 0.2) (layer "F.Cu") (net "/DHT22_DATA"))
 (segment (start 164 104.58) (end 161.54 104.58) (width 0.2) (layer "F.Cu") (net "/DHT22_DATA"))
 (segment (start 137.065686 122.5) (end 128.51 122.5) (width 0.2) (layer "F.Cu") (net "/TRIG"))
 (segment (start 176.97 124) (end 159.5 124) (width 0.2) (layer "F.Cu") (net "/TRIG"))
 (segment (start 128.51 122.5) (end 127.25 121.24) (width 0.2) (layer "F.Cu") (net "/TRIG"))
 (segment (start 159.5 124) (end 156 127.5) (width 0.2) (layer "F.Cu") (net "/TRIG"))
 (segment (start 182.5 127.46) (end 180.43 127.46) (width 0.2) (layer "F.Cu") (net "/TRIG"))
 (segment (start 156 132.5) (end 154.5 134) (width 0.2) (layer "F.Cu") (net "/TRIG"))
 (segment (start 154.5 134) (end 148.565686 134) (width 0.2) (layer "F.Cu") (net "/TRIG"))
 (segment (start 148.565686 134) (end 137.065686 122.5) (width 0.2) (layer "F.Cu") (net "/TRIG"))
 (segment (start 180.43 127.46) (end 176.97 124) (width 0.2) (layer "F.Cu") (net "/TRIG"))
 (segment (start 156 127.5) (end 156 132.5) (width 0.2) (layer "F.Cu") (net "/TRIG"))
 (segment (start 161.92 129) (end 161.92 131.5) (width 0.2) (layer "F.Cu") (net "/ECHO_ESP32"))
 (segment (start 134.2 126.32) (end 140.38 132.5) (width 0.2) (layer "F.Cu") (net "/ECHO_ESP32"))
 (segment (start 157 133) (end 157 130.25) (width 0.2) (layer "F.Cu") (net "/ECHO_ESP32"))
 (segment (start 155 135) (end 157 133) (width 0.2) (layer "F.Cu") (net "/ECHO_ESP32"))
 (segment (start 140.38 132.5) (end 145.5 132.5) (width 0.2) (layer "F.Cu") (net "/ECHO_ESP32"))
 (segment (start 161.92 126.5) (end 161.92 129) (width 0.2) (layer "F.Cu") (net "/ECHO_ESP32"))
 (segment (start 127.25 126.32) (end 134.2 126.32) (width 0.2) (layer "F.Cu") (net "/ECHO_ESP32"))
 (segment (start 148 135) (end 155 135) (width 0.2) (layer "F.Cu") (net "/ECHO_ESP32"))
 (segment (start 145.5 132.5) (end 148 135) (width 0.2) (layer "F.Cu") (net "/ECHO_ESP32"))
 (segment (start 157 130.25) (end 158.25 129) (width 0.2) (layer "F.Cu") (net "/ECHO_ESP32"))
 (segment (start 158.25 129) (end 161.92 129) (width 0.2) (layer "F.Cu") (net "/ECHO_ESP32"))
 (segment (start 173.5 126.5) (end 177 130) (width 0.2) (layer "F.Cu") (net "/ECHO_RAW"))
 (segment (start 177 130) (end 182.5 130) (width 0.2) (layer "F.Cu") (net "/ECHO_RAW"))
 (segment (start 172.08 126.5) (end 173.5 126.5) (width 0.2) (layer "F.Cu") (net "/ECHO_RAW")))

